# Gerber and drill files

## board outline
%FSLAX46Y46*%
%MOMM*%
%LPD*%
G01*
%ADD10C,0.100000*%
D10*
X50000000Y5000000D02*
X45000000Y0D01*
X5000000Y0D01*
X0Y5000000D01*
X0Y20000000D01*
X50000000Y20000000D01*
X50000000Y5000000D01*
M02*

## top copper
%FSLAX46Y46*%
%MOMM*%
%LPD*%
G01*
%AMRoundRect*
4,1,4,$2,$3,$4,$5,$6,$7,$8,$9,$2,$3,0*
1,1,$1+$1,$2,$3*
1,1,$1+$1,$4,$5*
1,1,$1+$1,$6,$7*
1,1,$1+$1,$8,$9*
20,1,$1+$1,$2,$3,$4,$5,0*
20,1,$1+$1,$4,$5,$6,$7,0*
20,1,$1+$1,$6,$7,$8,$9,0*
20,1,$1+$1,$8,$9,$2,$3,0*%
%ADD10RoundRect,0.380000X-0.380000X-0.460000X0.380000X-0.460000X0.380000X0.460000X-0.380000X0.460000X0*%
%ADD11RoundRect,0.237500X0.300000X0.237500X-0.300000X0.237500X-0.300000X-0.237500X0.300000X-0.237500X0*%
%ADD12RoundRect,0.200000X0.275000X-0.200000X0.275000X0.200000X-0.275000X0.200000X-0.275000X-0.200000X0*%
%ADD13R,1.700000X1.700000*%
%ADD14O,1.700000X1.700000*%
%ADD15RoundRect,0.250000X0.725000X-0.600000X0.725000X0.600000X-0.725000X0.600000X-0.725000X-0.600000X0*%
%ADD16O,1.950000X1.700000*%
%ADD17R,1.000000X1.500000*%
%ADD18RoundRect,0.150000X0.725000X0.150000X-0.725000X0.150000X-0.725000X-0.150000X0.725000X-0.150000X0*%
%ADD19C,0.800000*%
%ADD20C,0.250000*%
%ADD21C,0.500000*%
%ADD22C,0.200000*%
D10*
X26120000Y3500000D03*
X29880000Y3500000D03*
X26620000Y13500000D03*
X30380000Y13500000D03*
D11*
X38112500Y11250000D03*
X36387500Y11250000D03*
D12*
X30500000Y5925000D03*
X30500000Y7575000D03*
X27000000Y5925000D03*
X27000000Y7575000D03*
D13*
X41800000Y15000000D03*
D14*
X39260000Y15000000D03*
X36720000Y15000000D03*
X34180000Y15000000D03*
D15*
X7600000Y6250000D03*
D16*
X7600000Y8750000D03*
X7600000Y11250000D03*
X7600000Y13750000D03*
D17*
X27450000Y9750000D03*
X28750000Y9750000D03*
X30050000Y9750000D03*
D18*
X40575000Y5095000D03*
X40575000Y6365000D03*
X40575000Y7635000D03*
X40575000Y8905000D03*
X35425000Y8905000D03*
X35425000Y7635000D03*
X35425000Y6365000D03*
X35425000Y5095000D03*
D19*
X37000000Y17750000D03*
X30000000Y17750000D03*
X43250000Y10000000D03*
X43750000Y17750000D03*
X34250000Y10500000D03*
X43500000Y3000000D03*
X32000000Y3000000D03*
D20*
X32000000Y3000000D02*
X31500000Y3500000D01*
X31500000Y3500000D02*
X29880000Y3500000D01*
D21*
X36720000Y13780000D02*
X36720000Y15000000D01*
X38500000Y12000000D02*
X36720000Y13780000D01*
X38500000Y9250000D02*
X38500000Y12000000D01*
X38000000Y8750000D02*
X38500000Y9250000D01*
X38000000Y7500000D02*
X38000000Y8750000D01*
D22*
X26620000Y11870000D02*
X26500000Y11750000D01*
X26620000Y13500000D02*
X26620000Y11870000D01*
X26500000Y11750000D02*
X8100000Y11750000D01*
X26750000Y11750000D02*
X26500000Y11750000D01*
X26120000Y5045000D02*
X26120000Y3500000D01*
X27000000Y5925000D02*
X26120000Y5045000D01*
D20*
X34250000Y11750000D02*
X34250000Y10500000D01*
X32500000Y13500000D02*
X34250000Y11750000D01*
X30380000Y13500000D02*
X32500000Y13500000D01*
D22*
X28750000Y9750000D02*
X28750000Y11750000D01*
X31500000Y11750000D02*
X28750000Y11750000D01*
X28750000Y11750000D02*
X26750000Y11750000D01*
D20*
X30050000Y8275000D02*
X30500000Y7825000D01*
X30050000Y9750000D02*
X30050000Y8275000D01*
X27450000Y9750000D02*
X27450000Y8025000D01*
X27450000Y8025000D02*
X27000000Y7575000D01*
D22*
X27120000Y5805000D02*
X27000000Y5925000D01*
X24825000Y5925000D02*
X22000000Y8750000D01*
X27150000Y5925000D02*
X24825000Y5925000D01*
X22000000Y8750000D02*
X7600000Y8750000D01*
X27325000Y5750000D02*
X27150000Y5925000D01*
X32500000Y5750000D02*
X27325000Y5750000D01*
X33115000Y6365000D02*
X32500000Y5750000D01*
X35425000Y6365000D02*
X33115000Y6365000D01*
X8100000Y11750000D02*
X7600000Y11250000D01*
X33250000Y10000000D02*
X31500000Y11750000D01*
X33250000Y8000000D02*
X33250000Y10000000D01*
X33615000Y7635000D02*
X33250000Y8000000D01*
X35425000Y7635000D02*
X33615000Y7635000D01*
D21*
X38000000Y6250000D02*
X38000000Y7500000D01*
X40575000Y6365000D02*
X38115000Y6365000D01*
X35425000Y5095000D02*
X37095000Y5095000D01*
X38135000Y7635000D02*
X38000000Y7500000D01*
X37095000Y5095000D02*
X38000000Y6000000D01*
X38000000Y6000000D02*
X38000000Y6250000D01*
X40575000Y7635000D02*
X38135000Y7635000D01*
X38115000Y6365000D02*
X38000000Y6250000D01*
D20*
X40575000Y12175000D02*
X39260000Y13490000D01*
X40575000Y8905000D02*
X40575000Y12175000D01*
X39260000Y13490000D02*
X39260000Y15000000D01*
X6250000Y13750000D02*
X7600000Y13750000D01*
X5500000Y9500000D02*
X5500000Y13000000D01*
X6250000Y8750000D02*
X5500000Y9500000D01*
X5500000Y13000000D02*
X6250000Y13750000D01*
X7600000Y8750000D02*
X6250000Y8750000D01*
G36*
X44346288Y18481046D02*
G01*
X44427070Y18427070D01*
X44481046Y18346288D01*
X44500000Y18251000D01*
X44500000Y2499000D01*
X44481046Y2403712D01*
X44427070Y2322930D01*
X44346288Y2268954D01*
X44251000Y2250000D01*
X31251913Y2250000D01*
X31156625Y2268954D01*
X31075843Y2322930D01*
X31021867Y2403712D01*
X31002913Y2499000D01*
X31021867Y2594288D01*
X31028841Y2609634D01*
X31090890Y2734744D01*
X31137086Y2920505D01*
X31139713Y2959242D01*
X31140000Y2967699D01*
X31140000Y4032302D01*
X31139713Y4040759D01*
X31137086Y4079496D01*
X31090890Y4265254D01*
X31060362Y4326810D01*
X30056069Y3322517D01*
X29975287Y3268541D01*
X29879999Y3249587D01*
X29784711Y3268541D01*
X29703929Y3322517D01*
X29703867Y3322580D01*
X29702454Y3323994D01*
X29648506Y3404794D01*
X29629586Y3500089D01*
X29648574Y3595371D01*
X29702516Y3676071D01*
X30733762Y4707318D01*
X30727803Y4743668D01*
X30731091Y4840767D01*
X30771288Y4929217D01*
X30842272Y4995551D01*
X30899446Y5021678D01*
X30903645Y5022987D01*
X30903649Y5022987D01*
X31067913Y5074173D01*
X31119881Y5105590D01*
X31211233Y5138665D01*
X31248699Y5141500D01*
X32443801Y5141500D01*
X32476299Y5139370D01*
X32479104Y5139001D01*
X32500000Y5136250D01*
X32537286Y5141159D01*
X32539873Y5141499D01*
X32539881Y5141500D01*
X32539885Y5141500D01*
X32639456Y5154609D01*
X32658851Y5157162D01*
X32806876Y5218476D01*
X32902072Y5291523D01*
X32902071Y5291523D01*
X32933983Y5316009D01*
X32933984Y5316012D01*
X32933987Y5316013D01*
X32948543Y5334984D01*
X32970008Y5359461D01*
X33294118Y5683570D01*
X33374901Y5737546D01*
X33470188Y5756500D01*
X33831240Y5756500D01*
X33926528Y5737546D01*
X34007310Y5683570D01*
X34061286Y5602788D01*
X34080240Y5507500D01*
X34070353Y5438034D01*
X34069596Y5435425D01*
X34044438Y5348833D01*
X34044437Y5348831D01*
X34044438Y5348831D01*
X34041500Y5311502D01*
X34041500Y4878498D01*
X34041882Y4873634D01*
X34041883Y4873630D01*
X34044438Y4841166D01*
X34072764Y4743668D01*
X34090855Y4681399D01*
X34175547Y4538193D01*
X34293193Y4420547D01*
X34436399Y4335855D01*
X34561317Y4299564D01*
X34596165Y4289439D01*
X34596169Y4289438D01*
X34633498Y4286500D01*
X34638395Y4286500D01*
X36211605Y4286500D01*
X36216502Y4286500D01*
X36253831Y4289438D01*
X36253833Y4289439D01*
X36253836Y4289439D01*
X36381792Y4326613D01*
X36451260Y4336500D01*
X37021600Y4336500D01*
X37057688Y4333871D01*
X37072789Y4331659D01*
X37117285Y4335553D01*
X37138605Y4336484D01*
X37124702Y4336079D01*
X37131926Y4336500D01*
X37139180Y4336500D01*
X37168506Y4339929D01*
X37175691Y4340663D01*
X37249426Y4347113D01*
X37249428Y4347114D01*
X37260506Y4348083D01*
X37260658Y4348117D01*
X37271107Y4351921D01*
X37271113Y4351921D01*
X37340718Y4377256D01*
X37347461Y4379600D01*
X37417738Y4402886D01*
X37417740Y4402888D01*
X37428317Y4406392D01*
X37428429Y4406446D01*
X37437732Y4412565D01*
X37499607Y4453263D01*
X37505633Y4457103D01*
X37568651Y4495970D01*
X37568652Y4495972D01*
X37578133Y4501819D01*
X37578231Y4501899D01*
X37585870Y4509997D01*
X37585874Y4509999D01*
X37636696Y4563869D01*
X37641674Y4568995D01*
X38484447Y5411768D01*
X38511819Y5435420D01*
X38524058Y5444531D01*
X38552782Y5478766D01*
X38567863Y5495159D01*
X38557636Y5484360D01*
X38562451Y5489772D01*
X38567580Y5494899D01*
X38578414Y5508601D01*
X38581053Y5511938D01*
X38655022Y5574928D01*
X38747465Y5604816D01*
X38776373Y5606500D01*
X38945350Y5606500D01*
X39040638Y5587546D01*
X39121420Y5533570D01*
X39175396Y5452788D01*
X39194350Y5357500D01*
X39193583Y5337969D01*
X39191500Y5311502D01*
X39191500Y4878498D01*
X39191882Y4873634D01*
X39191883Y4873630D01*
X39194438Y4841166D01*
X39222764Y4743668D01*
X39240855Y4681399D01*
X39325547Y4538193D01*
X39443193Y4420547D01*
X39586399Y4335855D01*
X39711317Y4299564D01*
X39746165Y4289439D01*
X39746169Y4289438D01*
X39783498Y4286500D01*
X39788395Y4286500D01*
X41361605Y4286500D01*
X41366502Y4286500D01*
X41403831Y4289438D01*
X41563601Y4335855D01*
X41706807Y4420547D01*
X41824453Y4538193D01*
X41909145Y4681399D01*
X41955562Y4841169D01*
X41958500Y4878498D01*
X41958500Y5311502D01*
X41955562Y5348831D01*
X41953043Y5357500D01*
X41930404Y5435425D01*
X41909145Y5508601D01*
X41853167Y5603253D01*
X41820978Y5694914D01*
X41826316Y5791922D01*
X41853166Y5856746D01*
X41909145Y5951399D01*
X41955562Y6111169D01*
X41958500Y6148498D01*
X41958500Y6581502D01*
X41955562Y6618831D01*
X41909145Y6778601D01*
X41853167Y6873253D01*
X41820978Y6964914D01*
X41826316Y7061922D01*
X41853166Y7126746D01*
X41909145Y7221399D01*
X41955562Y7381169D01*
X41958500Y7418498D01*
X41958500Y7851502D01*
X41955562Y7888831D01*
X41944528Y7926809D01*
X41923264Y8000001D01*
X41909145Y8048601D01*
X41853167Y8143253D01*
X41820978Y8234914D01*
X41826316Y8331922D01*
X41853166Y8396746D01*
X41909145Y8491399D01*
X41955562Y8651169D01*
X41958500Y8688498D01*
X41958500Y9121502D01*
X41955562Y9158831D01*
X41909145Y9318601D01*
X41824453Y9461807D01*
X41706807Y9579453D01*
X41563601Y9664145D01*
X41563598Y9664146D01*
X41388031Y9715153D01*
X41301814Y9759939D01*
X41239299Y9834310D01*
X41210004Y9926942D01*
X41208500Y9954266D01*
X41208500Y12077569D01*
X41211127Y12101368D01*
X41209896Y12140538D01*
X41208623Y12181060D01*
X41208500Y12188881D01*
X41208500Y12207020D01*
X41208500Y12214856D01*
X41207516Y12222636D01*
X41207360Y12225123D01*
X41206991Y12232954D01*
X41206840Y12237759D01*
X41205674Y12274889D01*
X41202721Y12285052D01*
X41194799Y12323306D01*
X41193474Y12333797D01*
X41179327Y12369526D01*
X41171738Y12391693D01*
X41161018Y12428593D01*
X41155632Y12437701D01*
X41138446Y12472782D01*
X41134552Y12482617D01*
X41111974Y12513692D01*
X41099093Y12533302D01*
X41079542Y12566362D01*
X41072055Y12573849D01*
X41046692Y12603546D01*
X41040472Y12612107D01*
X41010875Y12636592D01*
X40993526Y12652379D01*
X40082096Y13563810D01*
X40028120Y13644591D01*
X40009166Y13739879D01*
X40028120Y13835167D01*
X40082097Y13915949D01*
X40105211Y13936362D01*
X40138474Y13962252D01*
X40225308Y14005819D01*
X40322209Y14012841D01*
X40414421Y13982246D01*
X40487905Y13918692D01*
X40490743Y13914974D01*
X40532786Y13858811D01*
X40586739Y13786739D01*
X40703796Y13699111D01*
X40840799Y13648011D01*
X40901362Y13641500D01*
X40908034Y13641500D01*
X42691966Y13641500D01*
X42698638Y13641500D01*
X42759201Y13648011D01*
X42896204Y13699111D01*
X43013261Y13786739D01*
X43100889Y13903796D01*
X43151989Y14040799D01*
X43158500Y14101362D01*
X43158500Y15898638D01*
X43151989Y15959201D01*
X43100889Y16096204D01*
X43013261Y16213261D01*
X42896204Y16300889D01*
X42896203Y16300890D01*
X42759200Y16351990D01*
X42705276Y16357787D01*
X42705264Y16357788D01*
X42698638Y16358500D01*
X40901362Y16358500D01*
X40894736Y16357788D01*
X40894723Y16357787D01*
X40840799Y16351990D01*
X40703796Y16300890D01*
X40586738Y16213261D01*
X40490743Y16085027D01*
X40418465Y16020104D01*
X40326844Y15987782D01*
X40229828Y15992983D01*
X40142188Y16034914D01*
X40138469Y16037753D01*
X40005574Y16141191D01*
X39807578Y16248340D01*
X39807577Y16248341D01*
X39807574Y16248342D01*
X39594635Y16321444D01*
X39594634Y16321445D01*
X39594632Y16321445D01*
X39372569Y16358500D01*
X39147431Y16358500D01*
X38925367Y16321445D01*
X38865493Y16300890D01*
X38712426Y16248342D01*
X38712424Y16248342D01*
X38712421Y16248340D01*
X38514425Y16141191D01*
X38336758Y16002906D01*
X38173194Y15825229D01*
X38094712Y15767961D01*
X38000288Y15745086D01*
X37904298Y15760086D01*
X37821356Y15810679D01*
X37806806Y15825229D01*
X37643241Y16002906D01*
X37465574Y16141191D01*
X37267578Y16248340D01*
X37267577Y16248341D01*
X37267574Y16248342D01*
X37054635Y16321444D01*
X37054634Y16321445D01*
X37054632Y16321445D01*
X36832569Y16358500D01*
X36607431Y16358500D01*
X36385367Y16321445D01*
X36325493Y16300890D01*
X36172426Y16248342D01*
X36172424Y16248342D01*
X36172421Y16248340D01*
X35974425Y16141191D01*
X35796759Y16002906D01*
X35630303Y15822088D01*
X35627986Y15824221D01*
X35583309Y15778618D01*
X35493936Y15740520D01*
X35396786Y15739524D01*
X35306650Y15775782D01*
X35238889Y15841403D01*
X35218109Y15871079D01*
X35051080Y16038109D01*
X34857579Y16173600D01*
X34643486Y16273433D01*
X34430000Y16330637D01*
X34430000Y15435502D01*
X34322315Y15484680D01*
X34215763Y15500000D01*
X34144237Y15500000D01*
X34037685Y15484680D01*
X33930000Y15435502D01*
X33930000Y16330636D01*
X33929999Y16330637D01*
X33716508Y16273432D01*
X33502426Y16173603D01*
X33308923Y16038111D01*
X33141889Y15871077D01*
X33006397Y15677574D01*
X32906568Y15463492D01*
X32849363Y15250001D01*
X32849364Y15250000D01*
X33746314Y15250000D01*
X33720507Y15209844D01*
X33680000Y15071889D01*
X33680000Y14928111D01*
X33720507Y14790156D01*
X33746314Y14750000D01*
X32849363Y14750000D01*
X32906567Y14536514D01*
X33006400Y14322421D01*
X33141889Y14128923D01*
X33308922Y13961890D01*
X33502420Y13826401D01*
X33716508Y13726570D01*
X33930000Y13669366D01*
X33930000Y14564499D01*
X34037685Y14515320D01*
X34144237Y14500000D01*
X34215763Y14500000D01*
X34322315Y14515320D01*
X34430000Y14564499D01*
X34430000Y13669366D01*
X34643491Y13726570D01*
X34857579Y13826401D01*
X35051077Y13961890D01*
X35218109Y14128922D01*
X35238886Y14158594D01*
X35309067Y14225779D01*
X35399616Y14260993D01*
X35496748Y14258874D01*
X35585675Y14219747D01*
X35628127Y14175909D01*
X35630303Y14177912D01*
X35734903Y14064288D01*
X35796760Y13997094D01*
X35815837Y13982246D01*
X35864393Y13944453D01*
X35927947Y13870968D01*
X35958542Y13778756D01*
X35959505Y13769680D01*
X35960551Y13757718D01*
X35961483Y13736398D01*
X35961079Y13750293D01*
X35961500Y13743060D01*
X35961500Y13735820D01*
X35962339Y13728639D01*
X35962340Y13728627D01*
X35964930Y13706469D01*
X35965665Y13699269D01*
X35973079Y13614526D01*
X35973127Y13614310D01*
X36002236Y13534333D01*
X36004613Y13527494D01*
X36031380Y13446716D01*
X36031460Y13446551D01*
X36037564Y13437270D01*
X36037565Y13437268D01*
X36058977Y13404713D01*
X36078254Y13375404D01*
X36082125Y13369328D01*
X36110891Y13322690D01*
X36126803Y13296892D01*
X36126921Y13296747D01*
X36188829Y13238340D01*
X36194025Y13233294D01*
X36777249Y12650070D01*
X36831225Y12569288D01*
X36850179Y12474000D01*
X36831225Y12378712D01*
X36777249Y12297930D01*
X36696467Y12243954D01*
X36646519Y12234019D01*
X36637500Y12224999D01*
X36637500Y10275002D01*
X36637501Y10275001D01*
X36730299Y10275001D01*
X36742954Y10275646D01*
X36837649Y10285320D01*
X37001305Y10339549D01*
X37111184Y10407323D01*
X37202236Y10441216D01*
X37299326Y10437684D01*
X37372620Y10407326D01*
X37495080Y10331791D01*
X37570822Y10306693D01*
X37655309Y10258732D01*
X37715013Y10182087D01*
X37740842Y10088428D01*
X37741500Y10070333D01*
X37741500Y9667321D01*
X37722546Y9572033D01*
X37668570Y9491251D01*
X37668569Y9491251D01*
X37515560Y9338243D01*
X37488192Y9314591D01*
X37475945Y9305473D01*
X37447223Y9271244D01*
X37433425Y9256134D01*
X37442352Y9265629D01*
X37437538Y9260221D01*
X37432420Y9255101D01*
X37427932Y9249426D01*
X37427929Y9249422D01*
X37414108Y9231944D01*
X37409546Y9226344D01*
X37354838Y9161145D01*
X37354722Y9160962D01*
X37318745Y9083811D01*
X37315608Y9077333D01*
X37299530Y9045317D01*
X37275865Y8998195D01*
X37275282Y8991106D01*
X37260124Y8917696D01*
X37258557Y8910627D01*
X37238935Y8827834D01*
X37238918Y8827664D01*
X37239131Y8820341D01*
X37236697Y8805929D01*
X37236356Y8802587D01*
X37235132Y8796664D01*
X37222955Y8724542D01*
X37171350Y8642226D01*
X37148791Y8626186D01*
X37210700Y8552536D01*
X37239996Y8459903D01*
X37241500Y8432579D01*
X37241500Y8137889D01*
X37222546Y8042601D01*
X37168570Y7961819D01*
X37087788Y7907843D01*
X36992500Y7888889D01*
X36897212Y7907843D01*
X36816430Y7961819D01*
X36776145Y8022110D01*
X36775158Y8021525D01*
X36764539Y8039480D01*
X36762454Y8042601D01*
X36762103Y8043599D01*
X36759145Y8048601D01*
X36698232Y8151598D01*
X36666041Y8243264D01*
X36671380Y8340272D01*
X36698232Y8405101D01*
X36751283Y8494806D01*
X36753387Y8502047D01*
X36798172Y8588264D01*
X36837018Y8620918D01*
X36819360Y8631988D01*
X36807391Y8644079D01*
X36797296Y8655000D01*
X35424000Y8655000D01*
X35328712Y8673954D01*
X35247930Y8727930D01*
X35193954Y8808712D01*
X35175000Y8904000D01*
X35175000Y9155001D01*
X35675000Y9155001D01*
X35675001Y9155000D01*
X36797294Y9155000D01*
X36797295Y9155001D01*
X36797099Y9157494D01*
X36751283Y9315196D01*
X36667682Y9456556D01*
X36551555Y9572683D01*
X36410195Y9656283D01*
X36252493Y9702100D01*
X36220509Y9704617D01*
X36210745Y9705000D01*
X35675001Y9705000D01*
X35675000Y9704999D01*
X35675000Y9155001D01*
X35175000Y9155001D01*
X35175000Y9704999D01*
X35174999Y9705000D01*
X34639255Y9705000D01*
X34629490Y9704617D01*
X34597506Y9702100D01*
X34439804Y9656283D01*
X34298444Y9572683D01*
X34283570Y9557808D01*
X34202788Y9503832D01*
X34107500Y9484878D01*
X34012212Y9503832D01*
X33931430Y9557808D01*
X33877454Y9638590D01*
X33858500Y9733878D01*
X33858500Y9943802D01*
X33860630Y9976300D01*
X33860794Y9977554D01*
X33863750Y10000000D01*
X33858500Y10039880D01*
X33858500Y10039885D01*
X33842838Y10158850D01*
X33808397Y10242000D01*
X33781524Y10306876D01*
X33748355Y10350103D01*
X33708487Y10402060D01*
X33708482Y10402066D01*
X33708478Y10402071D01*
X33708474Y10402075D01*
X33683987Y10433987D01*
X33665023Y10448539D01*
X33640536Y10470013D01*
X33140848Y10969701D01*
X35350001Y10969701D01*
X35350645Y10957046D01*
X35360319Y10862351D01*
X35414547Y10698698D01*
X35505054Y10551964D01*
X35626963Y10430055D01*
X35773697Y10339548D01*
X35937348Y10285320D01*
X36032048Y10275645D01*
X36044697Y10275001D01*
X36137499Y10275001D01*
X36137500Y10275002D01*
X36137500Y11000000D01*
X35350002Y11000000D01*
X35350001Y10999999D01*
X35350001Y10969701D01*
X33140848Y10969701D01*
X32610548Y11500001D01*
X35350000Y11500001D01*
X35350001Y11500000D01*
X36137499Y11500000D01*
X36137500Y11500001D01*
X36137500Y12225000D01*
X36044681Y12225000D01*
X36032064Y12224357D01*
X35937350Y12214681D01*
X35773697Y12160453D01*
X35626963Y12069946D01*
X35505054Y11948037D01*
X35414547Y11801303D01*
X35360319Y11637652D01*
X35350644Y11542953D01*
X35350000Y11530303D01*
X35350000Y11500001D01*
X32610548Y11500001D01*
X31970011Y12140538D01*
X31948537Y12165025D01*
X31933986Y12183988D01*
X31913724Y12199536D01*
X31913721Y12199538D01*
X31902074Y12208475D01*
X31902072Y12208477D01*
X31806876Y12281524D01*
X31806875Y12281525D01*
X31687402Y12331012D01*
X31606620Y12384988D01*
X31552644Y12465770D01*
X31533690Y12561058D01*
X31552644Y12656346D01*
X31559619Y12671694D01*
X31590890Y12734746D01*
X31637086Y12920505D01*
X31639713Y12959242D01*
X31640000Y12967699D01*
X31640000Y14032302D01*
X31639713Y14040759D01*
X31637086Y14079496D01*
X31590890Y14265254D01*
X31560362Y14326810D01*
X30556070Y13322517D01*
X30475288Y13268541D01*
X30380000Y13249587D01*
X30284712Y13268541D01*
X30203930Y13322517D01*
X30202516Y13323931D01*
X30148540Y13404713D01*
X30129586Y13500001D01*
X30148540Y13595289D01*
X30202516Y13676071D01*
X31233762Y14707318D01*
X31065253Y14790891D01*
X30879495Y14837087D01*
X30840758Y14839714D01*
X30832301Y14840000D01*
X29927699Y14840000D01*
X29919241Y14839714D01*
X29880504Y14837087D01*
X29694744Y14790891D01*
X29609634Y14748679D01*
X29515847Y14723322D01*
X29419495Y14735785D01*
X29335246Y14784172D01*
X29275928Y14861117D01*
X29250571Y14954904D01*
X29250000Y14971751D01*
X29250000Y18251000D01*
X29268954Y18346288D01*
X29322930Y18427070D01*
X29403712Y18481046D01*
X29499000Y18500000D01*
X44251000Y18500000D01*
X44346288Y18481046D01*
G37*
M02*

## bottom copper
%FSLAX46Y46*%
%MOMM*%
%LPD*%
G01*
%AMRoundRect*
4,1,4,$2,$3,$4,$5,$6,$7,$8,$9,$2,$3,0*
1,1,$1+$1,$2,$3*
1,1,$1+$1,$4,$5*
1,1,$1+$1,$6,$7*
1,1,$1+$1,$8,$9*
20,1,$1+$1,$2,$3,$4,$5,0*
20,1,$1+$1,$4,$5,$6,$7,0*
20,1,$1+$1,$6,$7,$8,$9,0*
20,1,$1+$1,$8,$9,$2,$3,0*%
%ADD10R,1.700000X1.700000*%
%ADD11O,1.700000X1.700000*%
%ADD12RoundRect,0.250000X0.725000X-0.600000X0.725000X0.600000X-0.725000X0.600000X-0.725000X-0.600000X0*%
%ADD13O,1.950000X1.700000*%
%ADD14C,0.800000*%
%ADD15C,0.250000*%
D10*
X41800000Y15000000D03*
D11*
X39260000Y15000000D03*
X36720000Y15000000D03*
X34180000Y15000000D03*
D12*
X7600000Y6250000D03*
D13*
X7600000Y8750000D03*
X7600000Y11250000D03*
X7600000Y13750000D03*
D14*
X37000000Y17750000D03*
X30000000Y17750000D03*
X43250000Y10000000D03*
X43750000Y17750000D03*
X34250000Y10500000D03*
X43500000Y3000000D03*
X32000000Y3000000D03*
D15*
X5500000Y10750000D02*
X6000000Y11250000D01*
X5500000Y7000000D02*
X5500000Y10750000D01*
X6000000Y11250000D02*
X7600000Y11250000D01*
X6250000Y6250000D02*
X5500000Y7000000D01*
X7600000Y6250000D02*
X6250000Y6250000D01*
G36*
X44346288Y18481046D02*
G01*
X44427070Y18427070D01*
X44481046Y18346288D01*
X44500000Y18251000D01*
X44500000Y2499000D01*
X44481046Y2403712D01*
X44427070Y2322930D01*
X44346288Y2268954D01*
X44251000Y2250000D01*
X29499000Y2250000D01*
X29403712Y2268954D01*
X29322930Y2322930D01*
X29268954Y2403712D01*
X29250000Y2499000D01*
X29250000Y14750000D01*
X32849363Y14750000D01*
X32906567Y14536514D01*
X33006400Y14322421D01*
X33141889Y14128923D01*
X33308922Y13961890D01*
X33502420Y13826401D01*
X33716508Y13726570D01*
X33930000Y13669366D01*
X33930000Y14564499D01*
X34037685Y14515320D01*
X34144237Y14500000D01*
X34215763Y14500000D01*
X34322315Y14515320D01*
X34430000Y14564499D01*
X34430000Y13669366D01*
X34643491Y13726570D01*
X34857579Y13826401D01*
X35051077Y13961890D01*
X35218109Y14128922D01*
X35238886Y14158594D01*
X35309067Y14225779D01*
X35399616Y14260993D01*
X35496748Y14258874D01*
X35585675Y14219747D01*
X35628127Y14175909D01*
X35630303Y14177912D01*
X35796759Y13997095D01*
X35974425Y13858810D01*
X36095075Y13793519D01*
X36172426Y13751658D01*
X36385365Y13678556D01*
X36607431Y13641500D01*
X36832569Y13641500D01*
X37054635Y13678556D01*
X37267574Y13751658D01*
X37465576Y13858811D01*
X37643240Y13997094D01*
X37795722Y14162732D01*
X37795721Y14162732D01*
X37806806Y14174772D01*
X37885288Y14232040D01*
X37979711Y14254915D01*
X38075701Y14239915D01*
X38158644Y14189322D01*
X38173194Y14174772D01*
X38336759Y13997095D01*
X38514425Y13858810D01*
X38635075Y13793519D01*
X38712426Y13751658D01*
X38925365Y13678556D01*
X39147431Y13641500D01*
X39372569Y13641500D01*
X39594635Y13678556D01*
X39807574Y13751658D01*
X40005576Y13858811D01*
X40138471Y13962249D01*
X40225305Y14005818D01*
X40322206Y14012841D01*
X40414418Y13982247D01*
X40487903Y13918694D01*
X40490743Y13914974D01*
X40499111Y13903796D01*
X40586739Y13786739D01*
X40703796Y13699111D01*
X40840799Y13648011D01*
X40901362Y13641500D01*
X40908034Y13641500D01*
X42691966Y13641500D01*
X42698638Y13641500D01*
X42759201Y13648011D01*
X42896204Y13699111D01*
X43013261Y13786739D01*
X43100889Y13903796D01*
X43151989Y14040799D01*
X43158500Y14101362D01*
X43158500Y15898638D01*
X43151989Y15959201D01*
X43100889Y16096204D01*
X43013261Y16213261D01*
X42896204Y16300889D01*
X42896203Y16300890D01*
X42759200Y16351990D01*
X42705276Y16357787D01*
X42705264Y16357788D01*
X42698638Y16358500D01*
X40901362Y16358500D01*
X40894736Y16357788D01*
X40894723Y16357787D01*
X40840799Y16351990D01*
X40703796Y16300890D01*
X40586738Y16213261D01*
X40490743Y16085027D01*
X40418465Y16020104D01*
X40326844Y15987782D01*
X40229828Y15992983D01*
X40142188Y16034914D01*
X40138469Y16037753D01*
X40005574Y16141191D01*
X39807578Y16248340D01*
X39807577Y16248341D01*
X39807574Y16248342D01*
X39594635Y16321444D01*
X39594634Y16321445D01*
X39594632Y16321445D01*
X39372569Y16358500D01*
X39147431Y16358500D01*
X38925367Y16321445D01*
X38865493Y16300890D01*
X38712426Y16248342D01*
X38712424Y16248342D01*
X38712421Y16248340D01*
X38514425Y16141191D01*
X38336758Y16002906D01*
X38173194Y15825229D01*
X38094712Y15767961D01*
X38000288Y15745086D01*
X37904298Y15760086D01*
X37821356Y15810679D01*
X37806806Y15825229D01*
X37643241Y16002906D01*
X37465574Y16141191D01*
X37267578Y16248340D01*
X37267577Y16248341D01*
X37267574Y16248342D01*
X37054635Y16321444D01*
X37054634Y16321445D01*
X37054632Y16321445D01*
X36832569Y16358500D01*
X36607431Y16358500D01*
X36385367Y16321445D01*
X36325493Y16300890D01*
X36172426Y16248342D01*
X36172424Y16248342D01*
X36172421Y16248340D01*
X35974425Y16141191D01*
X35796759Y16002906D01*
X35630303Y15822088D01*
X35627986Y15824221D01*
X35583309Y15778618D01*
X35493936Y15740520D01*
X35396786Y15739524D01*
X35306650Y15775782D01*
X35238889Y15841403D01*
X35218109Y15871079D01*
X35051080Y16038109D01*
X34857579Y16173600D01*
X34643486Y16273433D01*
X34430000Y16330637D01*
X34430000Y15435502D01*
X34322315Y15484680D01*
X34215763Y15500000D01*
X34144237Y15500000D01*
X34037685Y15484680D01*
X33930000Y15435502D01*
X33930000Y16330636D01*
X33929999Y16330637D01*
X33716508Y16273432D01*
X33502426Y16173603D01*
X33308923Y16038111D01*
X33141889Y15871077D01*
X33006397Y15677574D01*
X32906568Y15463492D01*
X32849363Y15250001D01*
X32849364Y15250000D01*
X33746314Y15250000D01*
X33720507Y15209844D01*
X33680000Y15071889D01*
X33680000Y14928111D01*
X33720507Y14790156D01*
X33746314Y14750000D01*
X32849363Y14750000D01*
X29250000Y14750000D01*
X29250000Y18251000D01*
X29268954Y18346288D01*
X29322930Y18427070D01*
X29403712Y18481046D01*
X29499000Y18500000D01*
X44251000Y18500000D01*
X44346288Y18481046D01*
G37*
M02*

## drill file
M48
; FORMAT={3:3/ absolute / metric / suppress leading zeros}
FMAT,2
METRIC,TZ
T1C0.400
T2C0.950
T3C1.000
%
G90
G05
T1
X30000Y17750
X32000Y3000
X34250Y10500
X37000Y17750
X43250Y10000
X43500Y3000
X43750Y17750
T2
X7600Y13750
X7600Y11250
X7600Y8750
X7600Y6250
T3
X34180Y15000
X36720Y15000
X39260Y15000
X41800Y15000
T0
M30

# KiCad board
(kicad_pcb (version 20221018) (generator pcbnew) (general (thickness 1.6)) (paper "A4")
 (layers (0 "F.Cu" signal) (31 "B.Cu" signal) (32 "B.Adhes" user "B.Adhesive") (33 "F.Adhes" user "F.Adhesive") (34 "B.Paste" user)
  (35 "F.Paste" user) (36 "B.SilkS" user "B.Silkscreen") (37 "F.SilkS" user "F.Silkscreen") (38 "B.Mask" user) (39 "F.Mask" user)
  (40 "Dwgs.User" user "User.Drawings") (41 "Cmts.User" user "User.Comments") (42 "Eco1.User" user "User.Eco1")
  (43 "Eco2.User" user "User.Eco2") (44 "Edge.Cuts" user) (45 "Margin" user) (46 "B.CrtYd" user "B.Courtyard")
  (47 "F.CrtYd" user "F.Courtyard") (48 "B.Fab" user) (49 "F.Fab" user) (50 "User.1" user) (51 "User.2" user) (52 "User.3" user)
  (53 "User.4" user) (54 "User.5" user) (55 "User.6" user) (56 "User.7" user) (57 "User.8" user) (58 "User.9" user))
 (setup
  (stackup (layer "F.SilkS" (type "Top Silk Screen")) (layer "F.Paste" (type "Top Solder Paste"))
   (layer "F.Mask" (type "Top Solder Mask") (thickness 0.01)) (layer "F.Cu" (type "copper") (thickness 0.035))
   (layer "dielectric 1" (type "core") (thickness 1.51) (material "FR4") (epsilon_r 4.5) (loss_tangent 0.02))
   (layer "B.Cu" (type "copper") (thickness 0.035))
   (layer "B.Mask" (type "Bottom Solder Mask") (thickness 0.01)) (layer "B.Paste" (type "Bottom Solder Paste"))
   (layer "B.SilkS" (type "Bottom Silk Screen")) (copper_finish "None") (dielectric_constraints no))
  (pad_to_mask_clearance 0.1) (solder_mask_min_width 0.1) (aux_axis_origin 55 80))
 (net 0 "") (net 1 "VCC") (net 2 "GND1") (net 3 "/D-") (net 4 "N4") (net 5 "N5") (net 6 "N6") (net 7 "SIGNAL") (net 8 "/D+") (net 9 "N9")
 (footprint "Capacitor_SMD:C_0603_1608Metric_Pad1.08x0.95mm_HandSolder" (layer "F.Cu") (at 92.25 68.75 180)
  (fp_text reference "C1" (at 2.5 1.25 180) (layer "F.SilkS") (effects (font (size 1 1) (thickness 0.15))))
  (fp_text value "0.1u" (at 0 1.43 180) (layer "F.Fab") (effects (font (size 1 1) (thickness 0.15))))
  (pad "1" smd roundrect (at -0.8625 0 180) (size 1.075 0.95) (layers "F.Cu" "F.Paste" "F.Mask") (roundrect_rratio 0.25) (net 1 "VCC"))
  (pad "2" smd roundrect (at 0.8625 0 180) (size 1.075 0.95) (layers "F.Cu" "F.Paste" "F.Mask") (roundrect_rratio 0.25) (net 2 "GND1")))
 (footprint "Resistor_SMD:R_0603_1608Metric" (layer "F.Cu") (at 85.5 73.25 90)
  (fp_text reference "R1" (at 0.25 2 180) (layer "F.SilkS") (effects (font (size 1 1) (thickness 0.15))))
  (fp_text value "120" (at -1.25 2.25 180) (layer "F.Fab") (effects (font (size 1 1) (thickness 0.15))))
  (pad "1" smd roundrect (at -0.825 0 90) (size 0.8 0.95) (layers "F.Cu" "F.Paste" "F.Mask") (roundrect_rratio 0.25) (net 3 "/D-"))
  (pad "2" smd roundrect (at 0.825 0 90) (size 0.8 0.95) (layers "F.Cu" "F.Paste" "F.Mask") (roundrect_rratio 0.25) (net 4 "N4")))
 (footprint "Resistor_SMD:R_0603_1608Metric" (layer "F.Cu") (at 82 73.25 90)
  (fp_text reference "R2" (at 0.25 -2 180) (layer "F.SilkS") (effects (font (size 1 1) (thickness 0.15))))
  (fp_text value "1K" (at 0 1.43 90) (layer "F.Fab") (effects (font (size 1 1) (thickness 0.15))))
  (pad "1" smd roundrect (at -0.825 0 90) (size 0.8 0.95) (layers "F.Cu" "F.Paste" "F.Mask") (roundrect_rratio 0.25) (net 3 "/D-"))
  (pad "2" smd roundrect (at 0.825 0 90) (size 0.8 0.95) (layers "F.Cu" "F.Paste" "F.Mask") (roundrect_rratio 0.25) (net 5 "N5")))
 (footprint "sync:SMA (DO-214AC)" (layer "F.Cu") (at 83 76.5)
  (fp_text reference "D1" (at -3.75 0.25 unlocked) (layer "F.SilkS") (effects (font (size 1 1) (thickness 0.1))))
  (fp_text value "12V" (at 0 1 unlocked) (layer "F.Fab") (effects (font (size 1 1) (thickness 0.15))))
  (pad "1" smd roundrect (at -1.88 0) (size 1.52 1.68) (layers "F.Cu" "F.Paste" "F.Mask") (roundrect_rratio 0.25) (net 3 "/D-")
   (thermal_bridge_angle 45))
  (pad "2" smd roundrect (at 1.88 0) (size 1.52 1.68) (layers "F.Cu" "F.Paste" "F.Mask") (roundrect_rratio 0.25) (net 2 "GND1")
   (thermal_bridge_angle 45)))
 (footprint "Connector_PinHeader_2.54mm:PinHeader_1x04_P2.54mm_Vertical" (layer "F.Cu") (at 96.8 65 -90)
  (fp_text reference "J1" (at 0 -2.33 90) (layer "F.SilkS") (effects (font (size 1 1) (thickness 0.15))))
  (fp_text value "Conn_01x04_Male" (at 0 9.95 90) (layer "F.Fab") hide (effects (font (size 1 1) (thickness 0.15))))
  (pad "1" thru_hole rect (at 0 0 270) (size 1.7 1.7) (drill 1) (layers "*.Cu" "*.Mask") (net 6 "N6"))
  (pad "2" thru_hole oval (at 0 2.54 270) (size 1.7 1.7) (drill 1) (layers "*.Cu" "*.Mask") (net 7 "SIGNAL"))
  (pad "3" thru_hole oval (at 0 5.08 270) (size 1.7 1.7) (drill 1) (layers "*.Cu" "*.Mask") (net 1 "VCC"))
  (pad "4" thru_hole oval (at 0 7.62 270) (size 1.7 1.7) (drill 1) (layers "*.Cu" "*.Mask") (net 2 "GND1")))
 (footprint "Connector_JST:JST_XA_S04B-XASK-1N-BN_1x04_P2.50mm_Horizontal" (layer "F.Cu") (at 62.6 73.75 90)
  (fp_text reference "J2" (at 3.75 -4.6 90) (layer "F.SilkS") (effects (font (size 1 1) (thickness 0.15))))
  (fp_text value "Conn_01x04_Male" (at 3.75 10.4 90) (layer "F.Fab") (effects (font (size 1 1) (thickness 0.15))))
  (pad "1" thru_hole roundrect (at 0 0 90) (size 1.7 1.95) (drill 0.95) (layers "*.Cu" "*.Mask") (roundrect_rratio 0.1470588235)
   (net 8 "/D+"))
  (pad "2" thru_hole oval (at 2.5 0 90) (size 1.7 1.95) (drill 0.95) (layers "*.Cu" "*.Mask") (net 3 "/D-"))
  (pad "3" thru_hole oval (at 5 0 90) (size 1.7 1.95) (drill 0.95) (layers "*.Cu" "*.Mask") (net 8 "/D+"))
  (pad "4" thru_hole oval (at 7.5 0 90) (size 1.7 1.95) (drill 0.95) (layers "*.Cu" "*.Mask") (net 3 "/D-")))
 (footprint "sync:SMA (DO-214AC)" (layer "F.Cu") (at 83.5 66.5)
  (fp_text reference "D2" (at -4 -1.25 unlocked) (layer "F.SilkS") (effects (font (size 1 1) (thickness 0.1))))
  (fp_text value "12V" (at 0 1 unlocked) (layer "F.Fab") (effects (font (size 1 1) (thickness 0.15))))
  (pad "1" smd roundrect (at -1.88 0) (size 1.52 1.68) (layers "F.Cu" "F.Paste" "F.Mask") (roundrect_rratio 0.25) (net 8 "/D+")
   (thermal_bridge_angle 45))
  (pad "2" smd roundrect (at 1.88 0) (size 1.52 1.68) (layers "F.Cu" "F.Paste" "F.Mask") (roundrect_rratio 0.25) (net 2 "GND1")
   (thermal_bridge_angle 45)))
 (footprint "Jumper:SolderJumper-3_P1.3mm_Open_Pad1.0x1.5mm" (layer "F.Cu") (at 83.75 70.25)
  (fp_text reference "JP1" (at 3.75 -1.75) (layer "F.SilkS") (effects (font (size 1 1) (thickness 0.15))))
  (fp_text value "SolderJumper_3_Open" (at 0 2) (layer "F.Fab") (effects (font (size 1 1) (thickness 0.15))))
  (pad "1" smd rect (at -1.3 0) (size 1 1.5) (layers "F.Cu" "F.Mask") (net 5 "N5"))
  (pad "2" smd rect (at 0 0) (size 1 1.5) (layers "F.Cu" "F.Mask") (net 8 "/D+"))
  (pad "3" smd rect (at 1.3 0) (size 1 1.5) (layers "F.Cu" "F.Mask") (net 4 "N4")))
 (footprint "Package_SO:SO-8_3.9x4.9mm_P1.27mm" (layer "F.Cu") (at 93 73 180)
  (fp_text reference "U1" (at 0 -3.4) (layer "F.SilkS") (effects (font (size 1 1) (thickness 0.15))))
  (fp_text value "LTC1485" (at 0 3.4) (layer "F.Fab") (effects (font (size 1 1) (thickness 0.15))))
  (pad "1" smd roundrect (at -2.575 -1.905 180) (size 1.75 0.6) (layers "F.Cu" "F.Paste" "F.Mask") (roundrect_rratio 0.25) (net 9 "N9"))
  (pad "2" smd roundrect (at -2.575 -0.635 180) (size 1.75 0.6) (layers "F.Cu" "F.Paste" "F.Mask") (roundrect_rratio 0.25) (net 1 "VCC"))
  (pad "3" smd roundrect (at -2.575 0.635 180) (size 1.75 0.6) (layers "F.Cu" "F.Paste" "F.Mask") (roundrect_rratio 0.25) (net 1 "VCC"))
  (pad "4" smd roundrect (at -2.575 1.905 180) (size 1.75 0.6) (layers "F.Cu" "F.Paste" "F.Mask") (roundrect_rratio 0.25) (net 7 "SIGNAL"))
  (pad "5" smd roundrect (at 2.575 1.905 180) (size 1.75 0.6) (layers "F.Cu" "F.Paste" "F.Mask") (roundrect_rratio 0.25) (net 2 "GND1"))
  (pad "6" smd roundrect (at 2.575 0.635 180) (size 1.75 0.6) (layers "F.Cu" "F.Paste" "F.Mask") (roundrect_rratio 0.25) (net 8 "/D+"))
  (pad "7" smd roundrect (at 2.575 -0.635 180) (size 1.75 0.6) (layers "F.Cu" "F.Paste" "F.Mask") (roundrect_rratio 0.25) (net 3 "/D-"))
  (pad "8" smd roundrect (at 2.575 -1.905 180) (size 1.75 0.6) (layers "F.Cu" "F.Paste" "F.Mask") (roundrect_rratio 0.25) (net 1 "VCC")))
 (gr_poly
  (pts (xy 105 75) (xy 100 80) (xy 60 80) (xy 55 75) (xy 55 60) (xy 105 60)) (stroke (width 0.1) (type solid)) (fill none)
  (layer "Edge.Cuts"))
 (segment (start 93 73.75) (end 93 72.5) (width 0.5) (layer "F.Cu") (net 1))
 (segment (start 95.575 73.635) (end 93.115 73.635) (width 0.5) (layer "F.Cu") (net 1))
 (segment (start 90.425 74.905) (end 92.095 74.905) (width 0.5) (layer "F.Cu") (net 1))
 (segment (start 93.135 72.365) (end 93 72.5) (width 0.5) (layer "F.Cu") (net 1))
 (segment (start 91.72 66.22) (end 91.72 65) (width 0.5) (layer "F.Cu") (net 1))
 (segment (start 93 72.5) (end 93 71.25) (width 0.5) (layer "F.Cu") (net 1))
 (segment (start 92.095 74.905) (end 93 74) (width 0.5) (layer "F.Cu") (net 1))
 (segment (start 93.5 68) (end 91.72 66.22) (width 0.5) (layer "F.Cu") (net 1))
 (segment (start 93.5 70.75) (end 93.5 68) (width 0.5) (layer "F.Cu") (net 1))
 (segment (start 93 74) (end 93 73.75) (width 0.5) (layer "F.Cu") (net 1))
 (segment (start 95.575 72.365) (end 93.135 72.365) (width 0.5) (layer "F.Cu") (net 1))
 (segment (start 93.115 73.635) (end 93 73.75) (width 0.5) (layer "F.Cu") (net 1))
 (segment (start 93 71.25) (end 93.5 70.75) (width 0.5) (layer "F.Cu") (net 1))
 (segment (start 87.5 66.5) (end 89.25 68.25) (width 0.25) (layer "F.Cu") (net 2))
 (segment (start 89.25 68.25) (end 89.25 69.5) (width 0.25) (layer "F.Cu") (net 2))
 (segment (start 85.38 66.5) (end 87.5 66.5) (width 0.25) (layer "F.Cu") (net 2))
 (segment (start 87 77) (end 86.5 76.5) (width 0.25) (layer "F.Cu") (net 2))
 (segment (start 86.5 76.5) (end 84.88 76.5) (width 0.25) (layer "F.Cu") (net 2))
 (via (at 98.25 70) (size 0.8) (drill 0.4) (layers "F.Cu" "B.Cu") (free) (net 2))
 (via (at 98.75 62.25) (size 0.8) (drill 0.4) (layers "F.Cu" "B.Cu") (free) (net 2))
 (via (at 89.25 69.5) (size 0.8) (drill 0.4) (layers "F.Cu" "B.Cu") (free) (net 2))
 (via (at 98.5 77) (size 0.8) (drill 0.4) (layers "F.Cu" "B.Cu") (free) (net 2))
 (via (at 85 62.25) (size 0.8) (drill 0.4) (layers "F.Cu" "B.Cu") (free) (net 2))
 (via (at 92 62.25) (size 0.8) (drill 0.4) (layers "F.Cu" "B.Cu") (free) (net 2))
 (via (at 87 77) (size 0.8) (drill 0.4) (layers "F.Cu" "B.Cu") (free) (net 2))
 (segment (start 95.575 67.825) (end 94.26 66.51) (width 0.25) (layer "F.Cu") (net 7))
 (segment (start 95.575 71.095) (end 95.575 67.825) (width 0.25) (layer "F.Cu") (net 7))
 (segment (start 94.26 66.51) (end 94.26 65) (width 0.25) (layer "F.Cu") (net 7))
 (segment (start 81.62 66.5) (end 81.62 68.13) (width 0.2) (layer "F.Cu") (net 8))
 (segment (start 81.75 68.25) (end 81.5 68.25) (width 0.2) (layer "F.Cu") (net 8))
 (segment (start 81.5 68.25) (end 63.1 68.25) (width 0.2) (layer "F.Cu") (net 8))
 (segment (start 88.25 70) (end 86.5 68.25) (width 0.2) (layer "F.Cu") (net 8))
 (segment (start 83.75 68.25) (end 81.75 68.25) (width 0.2) (layer "F.Cu") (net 8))
 (segment (start 83.75 70.25) (end 83.75 68.25) (width 0.2) (layer "F.Cu") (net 8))
 (segment (start 88.25 72) (end 88.25 70) (width 0.2) (layer "F.Cu") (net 8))
 (segment (start 81.62 68.13) (end 81.5 68.25) (width 0.2) (layer "F.Cu") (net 8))
 (segment (start 86.5 68.25) (end 83.75 68.25) (width 0.2) (layer "F.Cu") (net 8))
 (segment (start 88.615 72.365) (end 88.25 72) (width 0.2) (layer "F.Cu") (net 8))
 (segment (start 63.1 68.25) (end 62.6 68.75) (width 0.2) (layer "F.Cu") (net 8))
 (segment (start 90.425 72.365) (end 88.615 72.365) (width 0.2) (layer "F.Cu") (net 8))
 (segment (start 60.5 69.25) (end 61 68.75) (width 0.25) (layer "B.Cu") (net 8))
 (segment (start 60.5 73) (end 60.5 69.25) (width 0.25) (layer "B.Cu") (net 8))
 (segment (start 61 68.75) (end 62.6 68.75) (width 0.25) (layer "B.Cu") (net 8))
 (segment (start 61.25 73.75) (end 60.5 73) (width 0.25) (layer "B.Cu") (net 8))
 (segment (start 62.6 73.75) (end 61.25 73.75) (width 0.25) (layer "B.Cu") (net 8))
 (segment (start 61.25 66.25) (end 62.6 66.25) (width 0.25) (layer "F.Cu") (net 3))
 (segment (start 82.325 74.25) (end 82.15 74.075) (width 0.2) (layer "F.Cu") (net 3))
 (segment (start 88.115 73.635) (end 87.5 74.25) (width 0.2) (layer "F.Cu") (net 3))
 (segment (start 82 74.075) (end 81.12 74.955) (width 0.2) (layer "F.Cu") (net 3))
 (segment (start 81.12 74.955) (end 81.12 76.5) (width 0.2) (layer "F.Cu") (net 3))
 (segment (start 87.5 74.25) (end 82.325 74.25) (width 0.2) (layer "F.Cu") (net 3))
 (segment (start 82.12 74.195) (end 82 74.075) (width 0.2) (layer "F.Cu") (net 3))
 (segment (start 60.5 70.5) (end 60.5 67) (width 0.25) (layer "F.Cu") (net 3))
 (segment (start 61.25 71.25) (end 60.5 70.5) (width 0.25) (layer "F.Cu") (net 3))
 (segment (start 60.5 67) (end 61.25 66.25) (width 0.25) (layer "F.Cu") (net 3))
 (segment (start 82.15 74.075) (end 79.825 74.075) (width 0.2) (layer "F.Cu") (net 3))
 (segment (start 62.6 71.25) (end 61.25 71.25) (width 0.25) (layer "F.Cu") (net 3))
 (segment (start 77 71.25) (end 62.6 71.25) (width 0.2) (layer "F.Cu") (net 3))
 (segment (start 90.425 73.635) (end 88.115 73.635) (width 0.2) (layer "F.Cu") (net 3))
 (segment (start 79.825 74.075) (end 77 71.25) (width 0.2) (layer "F.Cu") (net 3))
 (segment (start 85.05 70.25) (end 85.05 71.725) (width 0.25) (layer "F.Cu") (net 4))
 (segment (start 85.05 71.725) (end 85.5 72.175) (width 0.25) (layer "F.Cu") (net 4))
 (segment (start 82.45 71.975) (end 82 72.425) (width 0.25) (layer "F.Cu") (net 5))
 (segment (start 82.45 70.25) (end 82.45 71.975) (width 0.25) (layer "F.Cu") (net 5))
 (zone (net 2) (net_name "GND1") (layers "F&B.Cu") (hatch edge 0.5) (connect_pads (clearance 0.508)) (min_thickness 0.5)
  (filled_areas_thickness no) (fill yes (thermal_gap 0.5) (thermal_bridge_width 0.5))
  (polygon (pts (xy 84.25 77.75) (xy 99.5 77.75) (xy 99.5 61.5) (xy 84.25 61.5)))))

